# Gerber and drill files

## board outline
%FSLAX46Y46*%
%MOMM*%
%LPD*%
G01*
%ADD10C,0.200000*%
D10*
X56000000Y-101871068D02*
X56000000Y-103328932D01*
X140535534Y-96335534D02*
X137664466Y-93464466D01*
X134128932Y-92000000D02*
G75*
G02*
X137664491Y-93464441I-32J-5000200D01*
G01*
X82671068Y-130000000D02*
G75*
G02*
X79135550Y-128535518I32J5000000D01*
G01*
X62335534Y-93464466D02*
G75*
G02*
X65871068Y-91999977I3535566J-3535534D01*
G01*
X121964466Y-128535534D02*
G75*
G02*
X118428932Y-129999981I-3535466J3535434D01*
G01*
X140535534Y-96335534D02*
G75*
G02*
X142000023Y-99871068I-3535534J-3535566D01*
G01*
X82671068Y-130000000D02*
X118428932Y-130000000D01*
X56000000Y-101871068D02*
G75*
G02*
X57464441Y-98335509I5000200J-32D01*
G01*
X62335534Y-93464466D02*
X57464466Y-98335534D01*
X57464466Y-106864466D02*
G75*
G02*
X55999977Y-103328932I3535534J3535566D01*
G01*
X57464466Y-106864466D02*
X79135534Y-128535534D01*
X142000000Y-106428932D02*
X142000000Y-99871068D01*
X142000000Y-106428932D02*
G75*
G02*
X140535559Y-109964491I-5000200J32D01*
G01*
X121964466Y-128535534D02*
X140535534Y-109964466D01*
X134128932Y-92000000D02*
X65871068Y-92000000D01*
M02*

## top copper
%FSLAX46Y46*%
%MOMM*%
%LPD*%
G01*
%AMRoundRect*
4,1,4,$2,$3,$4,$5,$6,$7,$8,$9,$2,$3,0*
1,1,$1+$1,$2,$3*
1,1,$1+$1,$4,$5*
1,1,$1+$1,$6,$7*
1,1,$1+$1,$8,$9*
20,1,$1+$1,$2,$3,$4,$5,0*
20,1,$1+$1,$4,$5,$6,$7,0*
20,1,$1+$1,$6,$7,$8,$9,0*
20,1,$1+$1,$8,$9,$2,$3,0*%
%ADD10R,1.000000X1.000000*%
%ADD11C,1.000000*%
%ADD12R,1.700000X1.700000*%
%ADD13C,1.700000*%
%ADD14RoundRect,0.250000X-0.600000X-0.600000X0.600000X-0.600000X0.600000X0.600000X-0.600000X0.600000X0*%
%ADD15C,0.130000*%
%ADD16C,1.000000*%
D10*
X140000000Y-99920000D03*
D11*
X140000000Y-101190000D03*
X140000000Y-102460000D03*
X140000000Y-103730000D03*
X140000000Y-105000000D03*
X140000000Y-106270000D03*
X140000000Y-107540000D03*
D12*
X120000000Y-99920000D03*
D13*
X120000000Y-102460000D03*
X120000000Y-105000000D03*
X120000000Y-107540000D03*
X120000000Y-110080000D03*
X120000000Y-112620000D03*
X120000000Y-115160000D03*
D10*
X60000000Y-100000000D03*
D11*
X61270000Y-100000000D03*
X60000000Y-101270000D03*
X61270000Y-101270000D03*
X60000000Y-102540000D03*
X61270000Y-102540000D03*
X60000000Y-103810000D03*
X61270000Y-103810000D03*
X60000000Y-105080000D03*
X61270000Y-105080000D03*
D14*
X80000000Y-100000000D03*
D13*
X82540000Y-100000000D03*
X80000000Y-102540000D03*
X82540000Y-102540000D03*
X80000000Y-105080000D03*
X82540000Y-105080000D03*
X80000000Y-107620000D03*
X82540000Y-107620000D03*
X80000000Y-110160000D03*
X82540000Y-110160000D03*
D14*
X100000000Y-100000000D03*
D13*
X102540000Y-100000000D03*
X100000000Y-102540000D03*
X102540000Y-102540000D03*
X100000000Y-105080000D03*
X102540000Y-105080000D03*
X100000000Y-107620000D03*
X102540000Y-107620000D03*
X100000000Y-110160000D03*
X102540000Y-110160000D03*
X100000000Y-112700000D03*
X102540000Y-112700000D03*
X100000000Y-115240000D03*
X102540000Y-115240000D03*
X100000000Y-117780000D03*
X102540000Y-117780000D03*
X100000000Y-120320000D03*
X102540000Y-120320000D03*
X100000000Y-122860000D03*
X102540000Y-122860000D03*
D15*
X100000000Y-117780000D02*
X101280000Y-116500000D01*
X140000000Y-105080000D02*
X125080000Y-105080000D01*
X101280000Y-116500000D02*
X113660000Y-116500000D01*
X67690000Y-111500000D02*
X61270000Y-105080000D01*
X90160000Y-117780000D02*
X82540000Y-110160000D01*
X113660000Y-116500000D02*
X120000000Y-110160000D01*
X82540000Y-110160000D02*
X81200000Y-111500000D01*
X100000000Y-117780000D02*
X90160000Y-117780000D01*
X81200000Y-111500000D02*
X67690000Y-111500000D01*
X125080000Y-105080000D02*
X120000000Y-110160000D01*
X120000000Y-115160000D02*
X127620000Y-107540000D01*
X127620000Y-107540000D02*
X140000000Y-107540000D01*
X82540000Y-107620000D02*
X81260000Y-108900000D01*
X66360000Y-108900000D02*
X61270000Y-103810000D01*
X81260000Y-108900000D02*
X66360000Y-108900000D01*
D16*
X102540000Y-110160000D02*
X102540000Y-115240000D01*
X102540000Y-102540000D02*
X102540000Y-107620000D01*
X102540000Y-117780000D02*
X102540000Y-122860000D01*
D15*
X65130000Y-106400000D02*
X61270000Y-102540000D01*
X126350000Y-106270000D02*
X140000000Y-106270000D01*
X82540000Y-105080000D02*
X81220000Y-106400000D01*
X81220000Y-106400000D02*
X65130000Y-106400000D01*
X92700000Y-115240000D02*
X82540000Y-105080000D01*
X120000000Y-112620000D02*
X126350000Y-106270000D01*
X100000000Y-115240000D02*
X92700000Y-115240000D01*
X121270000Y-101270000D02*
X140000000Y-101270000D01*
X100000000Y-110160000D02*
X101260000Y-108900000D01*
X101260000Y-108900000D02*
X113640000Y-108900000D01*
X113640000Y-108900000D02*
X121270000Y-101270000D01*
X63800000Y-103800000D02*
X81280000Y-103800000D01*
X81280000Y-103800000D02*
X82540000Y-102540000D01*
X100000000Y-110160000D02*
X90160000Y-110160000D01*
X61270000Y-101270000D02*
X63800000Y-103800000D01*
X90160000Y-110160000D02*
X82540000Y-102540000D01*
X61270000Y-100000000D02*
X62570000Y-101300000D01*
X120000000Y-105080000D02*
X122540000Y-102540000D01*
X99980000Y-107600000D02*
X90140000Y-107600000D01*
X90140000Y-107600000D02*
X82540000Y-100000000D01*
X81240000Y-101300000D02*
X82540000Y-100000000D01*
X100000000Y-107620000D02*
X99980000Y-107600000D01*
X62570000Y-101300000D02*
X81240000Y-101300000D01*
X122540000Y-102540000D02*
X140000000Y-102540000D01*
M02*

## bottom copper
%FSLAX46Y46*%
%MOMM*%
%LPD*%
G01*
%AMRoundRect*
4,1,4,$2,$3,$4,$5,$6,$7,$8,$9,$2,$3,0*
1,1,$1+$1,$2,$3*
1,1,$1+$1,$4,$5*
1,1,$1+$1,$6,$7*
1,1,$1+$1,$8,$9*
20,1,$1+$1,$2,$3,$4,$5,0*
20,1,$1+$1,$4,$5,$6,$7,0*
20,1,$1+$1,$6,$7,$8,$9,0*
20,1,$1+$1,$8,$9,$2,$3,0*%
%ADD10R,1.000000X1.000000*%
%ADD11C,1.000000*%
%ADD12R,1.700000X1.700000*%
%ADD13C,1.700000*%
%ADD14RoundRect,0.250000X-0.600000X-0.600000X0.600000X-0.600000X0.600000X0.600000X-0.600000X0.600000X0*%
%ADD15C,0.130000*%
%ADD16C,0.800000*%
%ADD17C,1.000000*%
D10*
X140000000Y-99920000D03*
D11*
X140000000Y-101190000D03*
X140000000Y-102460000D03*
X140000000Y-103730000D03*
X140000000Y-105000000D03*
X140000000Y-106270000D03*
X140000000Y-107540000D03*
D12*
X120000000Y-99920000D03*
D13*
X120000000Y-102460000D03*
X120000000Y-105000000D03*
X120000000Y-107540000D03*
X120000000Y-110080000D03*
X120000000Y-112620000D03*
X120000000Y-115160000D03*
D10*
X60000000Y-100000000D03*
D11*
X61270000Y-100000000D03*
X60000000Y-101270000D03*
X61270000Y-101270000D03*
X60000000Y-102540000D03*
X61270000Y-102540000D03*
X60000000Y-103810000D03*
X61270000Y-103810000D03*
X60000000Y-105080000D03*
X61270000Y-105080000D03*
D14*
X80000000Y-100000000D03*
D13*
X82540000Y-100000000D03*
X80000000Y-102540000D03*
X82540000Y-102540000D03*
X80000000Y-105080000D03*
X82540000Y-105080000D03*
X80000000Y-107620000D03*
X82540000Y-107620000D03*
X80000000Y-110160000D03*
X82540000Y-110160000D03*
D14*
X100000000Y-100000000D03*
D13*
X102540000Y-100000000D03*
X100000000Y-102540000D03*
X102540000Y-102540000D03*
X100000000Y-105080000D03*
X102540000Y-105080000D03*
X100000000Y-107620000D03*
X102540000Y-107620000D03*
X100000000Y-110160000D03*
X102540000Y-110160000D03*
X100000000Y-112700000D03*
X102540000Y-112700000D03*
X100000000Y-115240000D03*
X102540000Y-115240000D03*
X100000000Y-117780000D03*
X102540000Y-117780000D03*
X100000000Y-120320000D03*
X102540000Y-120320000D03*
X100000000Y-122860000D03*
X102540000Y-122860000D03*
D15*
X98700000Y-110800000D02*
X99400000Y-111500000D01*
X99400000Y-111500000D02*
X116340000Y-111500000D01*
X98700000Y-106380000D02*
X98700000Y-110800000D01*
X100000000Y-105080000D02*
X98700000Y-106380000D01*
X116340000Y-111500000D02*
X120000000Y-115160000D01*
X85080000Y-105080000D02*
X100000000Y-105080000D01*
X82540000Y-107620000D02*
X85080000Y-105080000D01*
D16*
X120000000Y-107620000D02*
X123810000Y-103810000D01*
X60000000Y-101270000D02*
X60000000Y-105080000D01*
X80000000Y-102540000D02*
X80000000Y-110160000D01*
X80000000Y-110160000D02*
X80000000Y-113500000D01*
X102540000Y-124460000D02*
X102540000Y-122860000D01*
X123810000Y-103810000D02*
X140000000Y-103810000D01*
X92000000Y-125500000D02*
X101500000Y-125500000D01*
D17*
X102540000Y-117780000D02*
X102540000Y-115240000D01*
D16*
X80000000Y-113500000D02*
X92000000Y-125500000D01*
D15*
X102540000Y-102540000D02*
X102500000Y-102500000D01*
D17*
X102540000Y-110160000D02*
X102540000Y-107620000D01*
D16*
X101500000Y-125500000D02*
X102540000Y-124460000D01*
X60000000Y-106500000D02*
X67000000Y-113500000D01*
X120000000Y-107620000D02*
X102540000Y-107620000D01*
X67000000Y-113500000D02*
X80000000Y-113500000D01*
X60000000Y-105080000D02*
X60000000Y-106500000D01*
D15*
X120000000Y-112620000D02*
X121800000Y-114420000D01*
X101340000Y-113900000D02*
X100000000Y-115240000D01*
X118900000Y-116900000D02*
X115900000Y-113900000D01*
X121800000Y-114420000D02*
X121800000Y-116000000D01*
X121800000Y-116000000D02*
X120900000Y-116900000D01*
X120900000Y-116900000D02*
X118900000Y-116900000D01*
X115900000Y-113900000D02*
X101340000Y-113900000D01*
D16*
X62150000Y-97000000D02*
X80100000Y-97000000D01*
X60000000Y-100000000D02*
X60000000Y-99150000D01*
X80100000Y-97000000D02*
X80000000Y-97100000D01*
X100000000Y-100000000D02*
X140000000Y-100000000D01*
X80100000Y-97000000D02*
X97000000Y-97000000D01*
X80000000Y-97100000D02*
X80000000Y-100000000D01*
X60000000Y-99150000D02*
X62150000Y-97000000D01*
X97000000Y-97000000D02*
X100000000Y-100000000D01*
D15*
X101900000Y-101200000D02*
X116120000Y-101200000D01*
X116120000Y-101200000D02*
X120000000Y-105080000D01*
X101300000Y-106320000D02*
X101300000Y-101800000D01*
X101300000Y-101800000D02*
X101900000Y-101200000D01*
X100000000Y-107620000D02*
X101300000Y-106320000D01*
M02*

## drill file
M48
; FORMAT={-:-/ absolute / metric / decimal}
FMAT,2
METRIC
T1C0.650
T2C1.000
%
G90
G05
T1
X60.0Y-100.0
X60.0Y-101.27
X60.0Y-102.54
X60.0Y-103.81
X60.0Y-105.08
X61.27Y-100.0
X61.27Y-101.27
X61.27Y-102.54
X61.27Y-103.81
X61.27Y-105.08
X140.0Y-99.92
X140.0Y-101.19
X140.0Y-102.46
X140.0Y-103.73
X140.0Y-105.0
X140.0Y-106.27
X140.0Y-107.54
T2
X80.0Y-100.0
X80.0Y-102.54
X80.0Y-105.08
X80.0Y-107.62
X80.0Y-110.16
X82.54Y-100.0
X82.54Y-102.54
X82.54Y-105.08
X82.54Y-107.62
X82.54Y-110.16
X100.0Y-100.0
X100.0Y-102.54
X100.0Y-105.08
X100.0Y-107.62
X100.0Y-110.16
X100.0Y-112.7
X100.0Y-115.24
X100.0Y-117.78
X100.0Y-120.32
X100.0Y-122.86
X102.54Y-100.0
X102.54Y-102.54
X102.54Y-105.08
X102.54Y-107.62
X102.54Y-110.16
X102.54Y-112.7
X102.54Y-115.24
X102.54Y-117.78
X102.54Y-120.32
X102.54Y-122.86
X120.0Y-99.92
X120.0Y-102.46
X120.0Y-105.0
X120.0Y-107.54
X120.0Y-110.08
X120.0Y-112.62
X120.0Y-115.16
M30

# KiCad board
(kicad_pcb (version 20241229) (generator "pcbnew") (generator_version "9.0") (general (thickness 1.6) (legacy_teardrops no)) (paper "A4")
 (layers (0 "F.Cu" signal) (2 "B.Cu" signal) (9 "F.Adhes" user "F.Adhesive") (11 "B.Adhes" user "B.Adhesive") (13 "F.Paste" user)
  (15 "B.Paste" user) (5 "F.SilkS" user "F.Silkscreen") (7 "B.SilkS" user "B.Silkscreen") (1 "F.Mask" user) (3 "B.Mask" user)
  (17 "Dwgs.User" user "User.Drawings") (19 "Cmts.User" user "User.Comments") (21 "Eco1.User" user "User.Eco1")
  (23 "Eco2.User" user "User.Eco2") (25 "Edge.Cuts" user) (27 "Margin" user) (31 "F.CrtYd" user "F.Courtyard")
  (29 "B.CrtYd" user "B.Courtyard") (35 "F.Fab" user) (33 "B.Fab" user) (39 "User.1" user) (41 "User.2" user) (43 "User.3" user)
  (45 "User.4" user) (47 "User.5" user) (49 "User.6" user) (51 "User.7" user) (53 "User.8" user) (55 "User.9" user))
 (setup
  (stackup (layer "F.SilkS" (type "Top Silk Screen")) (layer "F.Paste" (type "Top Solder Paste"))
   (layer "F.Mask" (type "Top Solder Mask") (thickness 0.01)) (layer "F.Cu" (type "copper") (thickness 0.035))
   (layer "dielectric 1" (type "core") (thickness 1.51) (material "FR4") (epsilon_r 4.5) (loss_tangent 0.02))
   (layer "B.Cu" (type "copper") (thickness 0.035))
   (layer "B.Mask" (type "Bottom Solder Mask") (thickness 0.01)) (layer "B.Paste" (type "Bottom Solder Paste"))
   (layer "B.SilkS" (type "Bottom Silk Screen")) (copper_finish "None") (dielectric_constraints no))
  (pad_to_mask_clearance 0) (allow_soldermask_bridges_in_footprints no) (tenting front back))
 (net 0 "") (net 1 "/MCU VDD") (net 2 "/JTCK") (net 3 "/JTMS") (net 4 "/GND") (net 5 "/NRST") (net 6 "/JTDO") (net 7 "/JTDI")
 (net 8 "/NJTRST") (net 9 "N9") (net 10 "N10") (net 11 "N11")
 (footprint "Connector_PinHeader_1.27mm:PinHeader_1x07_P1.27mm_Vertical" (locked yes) (layer "F.Cu") (at 140 99.92)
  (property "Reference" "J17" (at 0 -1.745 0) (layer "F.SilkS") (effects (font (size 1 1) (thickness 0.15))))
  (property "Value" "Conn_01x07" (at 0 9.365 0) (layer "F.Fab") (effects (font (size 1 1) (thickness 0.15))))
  (pad "1" thru_hole rect (at 0 0) (size 1 1) (drill 0.65) (layers "*.Cu" "*.Mask") (remove_unused_layers no) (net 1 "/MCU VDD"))
  (pad "2" thru_hole circle (at 0 1.27) (size 1 1) (drill 0.65) (layers "*.Cu" "*.Mask") (remove_unused_layers no) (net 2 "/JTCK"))
  (pad "3" thru_hole circle (at 0 2.54) (size 1 1) (drill 0.65) (layers "*.Cu" "*.Mask") (remove_unused_layers no) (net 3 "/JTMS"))
  (pad "4" thru_hole circle (at 0 3.81) (size 1 1) (drill 0.65) (layers "*.Cu" "*.Mask") (remove_unused_layers no) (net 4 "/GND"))
  (pad "5" thru_hole circle (at 0 5.08) (size 1 1) (drill 0.65) (layers "*.Cu" "*.Mask") (remove_unused_layers no) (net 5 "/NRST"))
  (pad "6" thru_hole circle (at 0 6.35) (size 1 1) (drill 0.65) (layers "*.Cu" "*.Mask") (remove_unused_layers no) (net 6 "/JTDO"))
  (pad "7" thru_hole circle (at 0 7.62) (size 1 1) (drill 0.65) (layers "*.Cu" "*.Mask") (remove_unused_layers no) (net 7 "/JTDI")))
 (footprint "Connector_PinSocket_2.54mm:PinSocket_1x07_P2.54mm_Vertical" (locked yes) (layer "F.Cu") (at 120 99.92)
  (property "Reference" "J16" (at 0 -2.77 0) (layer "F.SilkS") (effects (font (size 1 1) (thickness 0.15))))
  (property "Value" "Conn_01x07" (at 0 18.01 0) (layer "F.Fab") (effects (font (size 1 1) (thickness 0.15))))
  (pad "1" thru_hole rect (at 0 0) (size 1.7 1.7) (drill 1) (layers "*.Cu" "*.Mask") (remove_unused_layers no) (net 1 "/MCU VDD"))
  (pad "2" thru_hole circle (at 0 2.54) (size 1.7 1.7) (drill 1) (layers "*.Cu" "*.Mask") (remove_unused_layers no) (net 2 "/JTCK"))
  (pad "3" thru_hole circle (at 0 5.08) (size 1.7 1.7) (drill 1) (layers "*.Cu" "*.Mask") (remove_unused_layers no) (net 3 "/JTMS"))
  (pad "4" thru_hole circle (at 0 7.62) (size 1.7 1.7) (drill 1) (layers "*.Cu" "*.Mask") (remove_unused_layers no) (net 4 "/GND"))
  (pad "5" thru_hole circle (at 0 10.16) (size 1.7 1.7) (drill 1) (layers "*.Cu" "*.Mask") (remove_unused_layers no) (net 5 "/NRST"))
  (pad "6" thru_hole circle (at 0 12.7) (size 1.7 1.7) (drill 1) (layers "*.Cu" "*.Mask") (remove_unused_layers no) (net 6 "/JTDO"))
  (pad "7" thru_hole circle (at 0 15.24) (size 1.7 1.7) (drill 1) (layers "*.Cu" "*.Mask") (remove_unused_layers no) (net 7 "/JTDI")))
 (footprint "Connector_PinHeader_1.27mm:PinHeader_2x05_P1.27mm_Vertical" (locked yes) (layer "F.Cu") (at 60 100)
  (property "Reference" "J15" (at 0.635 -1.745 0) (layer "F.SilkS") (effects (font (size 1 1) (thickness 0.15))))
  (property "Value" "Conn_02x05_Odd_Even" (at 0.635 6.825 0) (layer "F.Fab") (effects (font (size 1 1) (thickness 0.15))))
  (pad "1" thru_hole rect (at 0 0) (size 1 1) (drill 0.65) (layers "*.Cu" "*.Mask") (remove_unused_layers no) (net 1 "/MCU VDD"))
  (pad "2" thru_hole circle (at 1.27 0) (size 1 1) (drill 0.65) (layers "*.Cu" "*.Mask") (remove_unused_layers no) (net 3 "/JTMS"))
  (pad "3" thru_hole circle (at 0 1.27) (size 1 1) (drill 0.65) (layers "*.Cu" "*.Mask") (remove_unused_layers no) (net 4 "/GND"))
  (pad "4" thru_hole circle (at 1.27 1.27) (size 1 1) (drill 0.65) (layers "*.Cu" "*.Mask") (remove_unused_layers no) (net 2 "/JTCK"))
  (pad "5" thru_hole circle (at 0 2.54) (size 1 1) (drill 0.65) (layers "*.Cu" "*.Mask") (remove_unused_layers no) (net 4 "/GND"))
  (pad "6" thru_hole circle (at 1.27 2.54) (size 1 1) (drill 0.65) (layers "*.Cu" "*.Mask") (remove_unused_layers no) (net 6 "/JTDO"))
  (pad "7" thru_hole circle (at 0 3.81) (size 1 1) (drill 0.65) (layers "*.Cu" "*.Mask") (remove_unused_layers no) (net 4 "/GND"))
  (pad "8" thru_hole circle (at 1.27 3.81) (size 1 1) (drill 0.65) (layers "*.Cu" "*.Mask") (remove_unused_layers no) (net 7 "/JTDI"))
  (pad "9" thru_hole circle (at 0 5.08) (size 1 1) (drill 0.65) (layers "*.Cu" "*.Mask") (remove_unused_layers no) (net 4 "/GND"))
  (pad "10" thru_hole circle (at 1.27 5.08) (size 1 1) (drill 0.65) (layers "*.Cu" "*.Mask") (remove_unused_layers no) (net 5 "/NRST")))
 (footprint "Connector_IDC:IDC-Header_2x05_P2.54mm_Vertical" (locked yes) (layer "F.Cu") (at 80 100)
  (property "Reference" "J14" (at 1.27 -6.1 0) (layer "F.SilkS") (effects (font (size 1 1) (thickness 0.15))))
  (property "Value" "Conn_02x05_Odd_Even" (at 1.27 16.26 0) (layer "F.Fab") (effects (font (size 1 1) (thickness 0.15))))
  (pad "1" thru_hole roundrect (at 0 0) (size 1.7 1.7) (drill 1) (layers "*.Cu" "*.Mask") (remove_unused_layers no)
   (roundrect_rratio 0.147059) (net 1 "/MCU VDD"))
  (pad "2" thru_hole circle (at 2.54 0) (size 1.7 1.7) (drill 1) (layers "*.Cu" "*.Mask") (remove_unused_layers no) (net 3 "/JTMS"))
  (pad "3" thru_hole circle (at 0 2.54) (size 1.7 1.7) (drill 1) (layers "*.Cu" "*.Mask") (remove_unused_layers no) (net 4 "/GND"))
  (pad "4" thru_hole circle (at 2.54 2.54) (size 1.7 1.7) (drill 1) (layers "*.Cu" "*.Mask") (remove_unused_layers no) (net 2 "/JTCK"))
  (pad "5" thru_hole circle (at 0 5.08) (size 1.7 1.7) (drill 1) (layers "*.Cu" "*.Mask") (remove_unused_layers no) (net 4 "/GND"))
  (pad "6" thru_hole circle (at 2.54 5.08) (size 1.7 1.7) (drill 1) (layers "*.Cu" "*.Mask") (remove_unused_layers no) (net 6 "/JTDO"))
  (pad "7" thru_hole circle (at 0 7.62) (size 1.7 1.7) (drill 1) (layers "*.Cu" "*.Mask") (remove_unused_layers no) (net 4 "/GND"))
  (pad "8" thru_hole circle (at 2.54 7.62) (size 1.7 1.7) (drill 1) (layers "*.Cu" "*.Mask") (remove_unused_layers no) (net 7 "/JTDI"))
  (pad "9" thru_hole circle (at 0 10.16) (size 1.7 1.7) (drill 1) (layers "*.Cu" "*.Mask") (remove_unused_layers no) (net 4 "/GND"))
  (pad "10" thru_hole circle (at 2.54 10.16) (size 1.7 1.7) (drill 1) (layers "*.Cu" "*.Mask") (remove_unused_layers no) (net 5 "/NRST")))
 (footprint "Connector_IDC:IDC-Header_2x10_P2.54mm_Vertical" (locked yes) (layer "F.Cu") (at 100 100)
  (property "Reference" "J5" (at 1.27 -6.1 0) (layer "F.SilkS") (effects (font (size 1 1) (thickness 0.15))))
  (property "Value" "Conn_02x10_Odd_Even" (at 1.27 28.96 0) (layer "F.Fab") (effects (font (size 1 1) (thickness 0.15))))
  (pad "1" thru_hole roundrect (at 0 0) (size 1.7 1.7) (drill 1) (layers "*.Cu" "*.Mask") (remove_unused_layers no)
   (roundrect_rratio 0.147059) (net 1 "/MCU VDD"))
  (pad "2" thru_hole circle (at 2.54 0) (size 1.7 1.7) (drill 1) (layers "*.Cu" "*.Mask") (remove_unused_layers no) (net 1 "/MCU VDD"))
  (pad "3" thru_hole circle (at 0 2.54) (size 1.7 1.7) (drill 1) (layers "*.Cu" "*.Mask") (remove_unused_layers no) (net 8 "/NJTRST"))
  (pad "4" thru_hole circle (at 2.54 2.54) (size 1.7 1.7) (drill 1) (layers "*.Cu" "*.Mask") (remove_unused_layers no) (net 4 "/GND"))
  (pad "5" thru_hole circle (at 0 5.08) (size 1.7 1.7) (drill 1) (layers "*.Cu" "*.Mask") (remove_unused_layers no) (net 7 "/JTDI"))
  (pad "6" thru_hole circle (at 2.54 5.08) (size 1.7 1.7) (drill 1) (layers "*.Cu" "*.Mask") (remove_unused_layers no) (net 4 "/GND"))
  (pad "7" thru_hole circle (at 0 7.62) (size 1.7 1.7) (drill 1) (layers "*.Cu" "*.Mask") (remove_unused_layers no) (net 3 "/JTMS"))
  (pad "8" thru_hole circle (at 2.54 7.62) (size 1.7 1.7) (drill 1) (layers "*.Cu" "*.Mask") (remove_unused_layers no) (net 4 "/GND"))
  (pad "9" thru_hole circle (at 0 10.16) (size 1.7 1.7) (drill 1) (layers "*.Cu" "*.Mask") (remove_unused_layers no) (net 2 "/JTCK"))
  (pad "10" thru_hole circle (at 2.54 10.16) (size 1.7 1.7) (drill 1) (layers "*.Cu" "*.Mask") (remove_unused_layers no) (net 4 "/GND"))
  (pad "11" thru_hole circle (at 0 12.7) (size 1.7 1.7) (drill 1) (layers "*.Cu" "*.Mask") (remove_unused_layers no) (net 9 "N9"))
  (pad "12" thru_hole circle (at 2.54 12.7) (size 1.7 1.7) (drill 1) (layers "*.Cu" "*.Mask") (remove_unused_layers no) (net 4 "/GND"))
  (pad "13" thru_hole circle (at 0 15.24) (size 1.7 1.7) (drill 1) (layers "*.Cu" "*.Mask") (remove_unused_layers no) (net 6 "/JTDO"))
  (pad "14" thru_hole circle (at 2.54 15.24) (size 1.7 1.7) (drill 1) (layers "*.Cu" "*.Mask") (remove_unused_layers no) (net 4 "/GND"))
  (pad "15" thru_hole circle (at 0 17.78) (size 1.7 1.7) (drill 1) (layers "*.Cu" "*.Mask") (remove_unused_layers no) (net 5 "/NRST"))
  (pad "16" thru_hole circle (at 2.54 17.78) (size 1.7 1.7) (drill 1) (layers "*.Cu" "*.Mask") (remove_unused_layers no) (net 4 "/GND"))
  (pad "17" thru_hole circle (at 0 20.32) (size 1.7 1.7) (drill 1) (layers "*.Cu" "*.Mask") (remove_unused_layers no) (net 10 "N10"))
  (pad "18" thru_hole circle (at 2.54 20.32) (size 1.7 1.7) (drill 1) (layers "*.Cu" "*.Mask") (remove_unused_layers no) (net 4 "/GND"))
  (pad "19" thru_hole circle (at 0 22.86) (size 1.7 1.7) (drill 1) (layers "*.Cu" "*.Mask") (remove_unused_layers no) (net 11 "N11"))
  (pad "20" thru_hole circle (at 2.54 22.86) (size 1.7 1.7) (drill 1) (layers "*.Cu" "*.Mask") (remove_unused_layers no) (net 4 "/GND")))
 (gr_line (start 56 101.871068) (end 56 103.328932) (stroke (width 0.2) (type default)) (locked yes) (layer "Edge.Cuts"))
 (gr_line (start 140.535534 96.335534) (end 137.664466 93.464466) (stroke (width 0.2) (type default)) (locked yes) (layer "Edge.Cuts"))
 (gr_arc (start 134.128932 92) (mid 136.042342 92.380613) (end 137.664466 93.464466) (stroke (width 0.2) (type default)) (locked yes)
  (layer "Edge.Cuts"))
 (gr_arc (start 82.671068 130) (mid 80.757651 129.619398) (end 79.135534 128.535534) (stroke (width 0.2) (type default)) (locked yes)
  (layer "Edge.Cuts"))
 (gr_arc (start 62.335534 93.464466) (mid 63.957651 92.380602) (end 65.871068 92) (stroke (width 0.2) (type default)) (locked yes)
  (layer "Edge.Cuts"))
 (gr_arc (start 121.964466 128.535534) (mid 120.342351 129.619408) (end 118.428932 130) (stroke (width 0.2) (type default)) (locked yes)
  (layer "Edge.Cuts"))
 (gr_arc (start 140.535534 96.335534) (mid 141.619398 97.957651) (end 142 99.871068) (stroke (width 0.2) (type default)) (locked yes)
  (layer "Edge.Cuts"))
 (gr_line (start 82.671068 130) (end 118.428932 130) (stroke (width 0.2) (type default)) (locked yes) (layer "Edge.Cuts"))
 (gr_arc (start 56 101.871068) (mid 56.380613 99.957658) (end 57.464466 98.335534) (stroke (width 0.2) (type default)) (locked yes)
  (layer "Edge.Cuts"))
 (gr_line (start 62.335534 93.464466) (end 57.464466 98.335534) (stroke (width 0.2) (type default)) (locked yes) (layer "Edge.Cuts"))
 (gr_arc (start 57.464466 106.864466) (mid 56.380602 105.242349) (end 56 103.328932) (stroke (width 0.2) (type default)) (locked yes)
  (layer "Edge.Cuts"))
 (gr_line (start 57.464466 106.864466) (end 79.135534 128.535534) (stroke (width 0.2) (type default)) (locked yes) (layer "Edge.Cuts"))
 (gr_line (start 142 106.428932) (end 142 99.871068) (stroke (width 0.2) (type default)) (locked yes) (layer "Edge.Cuts"))
 (gr_arc (start 142 106.428932) (mid 141.619387 108.342342) (end 140.535534 109.964466) (stroke (width 0.2) (type default)) (locked yes)
  (layer "Edge.Cuts"))
 (gr_line (start 121.964466 128.535534) (end 140.535534 109.964466) (stroke (width 0.2) (type default)) (locked yes) (layer "Edge.Cuts"))
 (gr_line (start 134.128932 92) (end 65.871068 92) (stroke (width 0.2) (type default)) (locked yes) (layer "Edge.Cuts"))
 (segment (start 100 117.78) (end 101.28 116.5) (width 0.13) (locked yes) (layer "F.Cu") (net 5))
 (segment (start 140 105.08) (end 125.08 105.08) (width 0.13) (locked yes) (layer "F.Cu") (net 5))
 (segment (start 101.28 116.5) (end 113.66 116.5) (width 0.13) (locked yes) (layer "F.Cu") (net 5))
 (segment (start 67.69 111.5) (end 61.27 105.08) (width 0.13) (locked yes) (layer "F.Cu") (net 5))
 (segment (start 90.16 117.78) (end 82.54 110.16) (width 0.13) (locked yes) (layer "F.Cu") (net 5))
 (segment (start 113.66 116.5) (end 120 110.16) (width 0.13) (locked yes) (layer "F.Cu") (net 5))
 (segment (start 82.54 110.16) (end 81.2 111.5) (width 0.13) (locked yes) (layer "F.Cu") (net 5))
 (segment (start 100 117.78) (end 90.16 117.78) (width 0.13) (locked yes) (layer "F.Cu") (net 5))
 (segment (start 81.2 111.5) (end 67.69 111.5) (width 0.13) (locked yes) (layer "F.Cu") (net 5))
 (segment (start 125.08 105.08) (end 120 110.16) (width 0.13) (locked yes) (layer "F.Cu") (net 5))
 (segment (start 120 115.16) (end 127.62 107.54) (width 0.13) (locked yes) (layer "F.Cu") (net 7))
 (segment (start 127.62 107.54) (end 140 107.54) (width 0.13) (locked yes) (layer "F.Cu") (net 7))
 (segment (start 82.54 107.62) (end 81.26 108.9) (width 0.13) (locked yes) (layer "F.Cu") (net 7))
 (segment (start 66.36 108.9) (end 61.27 103.81) (width 0.13) (locked yes) (layer "F.Cu") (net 7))
 (segment (start 81.26 108.9) (end 66.36 108.9) (width 0.13) (locked yes) (layer "F.Cu") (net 7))
 (segment (start 98.7 110.8) (end 99.4 111.5) (width 0.13) (locked yes) (layer "B.Cu") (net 7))
 (segment (start 99.4 111.5) (end 116.34 111.5) (width 0.13) (locked yes) (layer "B.Cu") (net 7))
 (segment (start 98.7 106.38) (end 98.7 110.8) (width 0.13) (locked yes) (layer "B.Cu") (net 7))
 (segment (start 100 105.08) (end 98.7 106.38) (width 0.13) (locked yes) (layer "B.Cu") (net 7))
 (segment (start 116.34 111.5) (end 120 115.16) (width 0.13) (locked yes) (layer "B.Cu") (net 7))
 (segment (start 85.08 105.08) (end 100 105.08) (width 0.13) (locked yes) (layer "B.Cu") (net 7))
 (segment (start 82.54 107.62) (end 85.08 105.08) (width 0.13) (locked yes) (layer "B.Cu") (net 7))
 (segment (start 102.54 110.16) (end 102.54 115.24) (width 1) (locked yes) (layer "F.Cu") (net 4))
 (segment (start 102.54 102.54) (end 102.54 107.62) (width 1) (locked yes) (layer "F.Cu") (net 4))
 (segment (start 102.54 117.78) (end 102.54 122.86) (width 1) (locked yes) (layer "F.Cu") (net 4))
 (segment (start 120 107.62) (end 123.81 103.81) (width 0.8) (locked yes) (layer "B.Cu") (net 4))
 (segment (start 60 101.27) (end 60 105.08) (width 0.8) (locked yes) (layer "B.Cu") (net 4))
 (segment (start 80 102.54) (end 80 110.16) (width 0.8) (locked yes) (layer "B.Cu") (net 4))
 (segment (start 80 110.16) (end 80 113.5) (width 0.8) (locked yes) (layer "B.Cu") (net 4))
 (segment (start 102.54 124.46) (end 102.54 122.86) (width 0.8) (locked yes) (layer "B.Cu") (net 4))
 (segment (start 123.81 103.81) (end 140 103.81) (width 0.8) (locked yes) (layer "B.Cu") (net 4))
 (segment (start 92 125.5) (end 101.5 125.5) (width 0.8) (locked yes) (layer "B.Cu") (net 4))
 (segment (start 102.54 117.78) (end 102.54 115.24) (width 1) (locked yes) (layer "B.Cu") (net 4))
 (segment (start 80 113.5) (end 92 125.5) (width 0.8) (locked yes) (layer "B.Cu") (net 4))
 (segment (start 102.54 102.54) (end 102.5 102.5) (width 0.13) (locked yes) (layer "B.Cu") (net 4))
 (segment (start 102.54 110.16) (end 102.54 107.62) (width 1) (locked yes) (layer "B.Cu") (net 4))
 (segment (start 101.5 125.5) (end 102.54 124.46) (width 0.8) (locked yes) (layer "B.Cu") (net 4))
 (segment (start 60 106.5) (end 67 113.5) (width 0.8) (locked yes) (layer "B.Cu") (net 4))
 (segment (start 120 107.62) (end 102.54 107.62) (width 0.8) (locked yes) (layer "B.Cu") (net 4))
 (segment (start 67 113.5) (end 80 113.5) (width 0.8) (locked yes) (layer "B.Cu") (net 4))
 (segment (start 60 105.08) (end 60 106.5) (width 0.8) (locked yes) (layer "B.Cu") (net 4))
 (segment (start 65.13 106.4) (end 61.27 102.54) (width 0.13) (locked yes) (layer "F.Cu") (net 6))
 (segment (start 126.35 106.27) (end 140 106.27) (width 0.13) (locked yes) (layer "F.Cu") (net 6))
 (segment (start 82.54 105.08) (end 81.22 106.4) (width 0.13) (locked yes) (layer "F.Cu") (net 6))
 (segment (start 81.22 106.4) (end 65.13 106.4) (width 0.13) (locked yes) (layer "F.Cu") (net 6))
 (segment (start 92.7 115.24) (end 82.54 105.08) (width 0.13) (locked yes) (layer "F.Cu") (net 6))
 (segment (start 120 112.62) (end 126.35 106.27) (width 0.13) (locked yes) (layer "F.Cu") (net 6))
 (segment (start 100 115.24) (end 92.7 115.24) (width 0.13) (locked yes) (layer "F.Cu") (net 6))
 (segment (start 120 112.62) (end 121.8 114.42) (width 0.13) (locked yes) (layer "B.Cu") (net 6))
 (segment (start 101.34 113.9) (end 100 115.24) (width 0.13) (locked yes) (layer "B.Cu") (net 6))
 (segment (start 118.9 116.9) (end 115.9 113.9) (width 0.13) (locked yes) (layer "B.Cu") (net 6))
 (segment (start 121.8 114.42) (end 121.8 116) (width 0.13) (locked yes) (layer "B.Cu") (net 6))
 (segment (start 121.8 116) (end 120.9 116.9) (width 0.13) (locked yes) (layer "B.Cu") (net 6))
 (segment (start 120.9 116.9) (end 118.9 116.9) (width 0.13) (locked yes) (layer "B.Cu") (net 6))
 (segment (start 115.9 113.9) (end 101.34 113.9) (width 0.13) (locked yes) (layer "B.Cu") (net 6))
 (segment (start 121.27 101.27) (end 140 101.27) (width 0.13) (locked yes) (layer "F.Cu") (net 2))
 (segment (start 100 110.16) (end 101.26 108.9) (width 0.13) (locked yes) (layer "F.Cu") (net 2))
 (segment (start 101.26 108.9) (end 113.64 108.9) (width 0.13) (locked yes) (layer "F.Cu") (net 2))
 (segment (start 113.64 108.9) (end 121.27 101.27) (width 0.13) (locked yes) (layer "F.Cu") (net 2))
 (segment (start 63.8 103.8) (end 81.28 103.8) (width 0.13) (locked yes) (layer "F.Cu") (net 2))
 (segment (start 81.28 103.8) (end 82.54 102.54) (width 0.13) (locked yes) (layer "F.Cu") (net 2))
 (segment (start 100 110.16) (end 90.16 110.16) (width 0.13) (locked yes) (layer "F.Cu") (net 2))
 (segment (start 61.27 101.27) (end 63.8 103.8) (width 0.13) (locked yes) (layer "F.Cu") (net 2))
 (segment (start 90.16 110.16) (end 82.54 102.54) (width 0.13) (locked yes) (layer "F.Cu") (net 2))
 (segment (start 62.15 97) (end 80.1 97) (width 0.8) (locked yes) (layer "B.Cu") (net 1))
 (segment (start 60 100) (end 60 99.15) (width 0.8) (locked yes) (layer "B.Cu") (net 1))
 (segment (start 80.1 97) (end 80 97.1) (width 0.8) (locked yes) (layer "B.Cu") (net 1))
 (segment (start 100 100) (end 140 100) (width 0.8) (locked yes) (layer "B.Cu") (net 1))
 (segment (start 80.1 97) (end 97 97) (width 0.8) (locked yes) (layer "B.Cu") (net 1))
 (segment (start 80 97.1) (end 80 100) (width 0.8) (locked yes) (layer "B.Cu") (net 1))
 (segment (start 60 99.15) (end 62.15 97) (width 0.8) (locked yes) (layer "B.Cu") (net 1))
 (segment (start 97 97) (end 100 100) (width 0.8) (locked yes) (layer "B.Cu") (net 1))
 (segment (start 61.27 100) (end 62.57 101.3) (width 0.13) (locked yes) (layer "F.Cu") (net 3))
 (segment (start 120 105.08) (end 122.54 102.54) (width 0.13) (locked yes) (layer "F.Cu") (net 3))
 (segment (start 99.98 107.6) (end 90.14 107.6) (width 0.13) (locked yes) (layer "F.Cu") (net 3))
 (segment (start 90.14 107.6) (end 82.54 100) (width 0.13) (locked yes) (layer "F.Cu") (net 3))
 (segment (start 81.24 101.3) (end 82.54 100) (width 0.13) (locked yes) (layer "F.Cu") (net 3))
 (segment (start 100 107.62) (end 99.98 107.6) (width 0.13) (locked yes) (layer "F.Cu") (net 3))
 (segment (start 62.57 101.3) (end 81.24 101.3) (width 0.13) (locked yes) (layer "F.Cu") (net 3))
 (segment (start 122.54 102.54) (end 140 102.54) (width 0.13) (locked yes) (layer "F.Cu") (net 3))
 (segment (start 101.9 101.2) (end 116.12 101.2) (width 0.13) (locked yes) (layer "B.Cu") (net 3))
 (segment (start 116.12 101.2) (end 120 105.08) (width 0.13) (locked yes) (layer "B.Cu") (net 3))
 (segment (start 101.3 106.32) (end 101.3 101.8) (width 0.13) (locked yes) (layer "B.Cu") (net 3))
 (segment (start 101.3 101.8) (end 101.9 101.2) (width 0.13) (locked yes) (layer "B.Cu") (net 3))
 (segment (start 100 107.62) (end 101.3 106.32) (width 0.13) (locked yes) (layer "B.Cu") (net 3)))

